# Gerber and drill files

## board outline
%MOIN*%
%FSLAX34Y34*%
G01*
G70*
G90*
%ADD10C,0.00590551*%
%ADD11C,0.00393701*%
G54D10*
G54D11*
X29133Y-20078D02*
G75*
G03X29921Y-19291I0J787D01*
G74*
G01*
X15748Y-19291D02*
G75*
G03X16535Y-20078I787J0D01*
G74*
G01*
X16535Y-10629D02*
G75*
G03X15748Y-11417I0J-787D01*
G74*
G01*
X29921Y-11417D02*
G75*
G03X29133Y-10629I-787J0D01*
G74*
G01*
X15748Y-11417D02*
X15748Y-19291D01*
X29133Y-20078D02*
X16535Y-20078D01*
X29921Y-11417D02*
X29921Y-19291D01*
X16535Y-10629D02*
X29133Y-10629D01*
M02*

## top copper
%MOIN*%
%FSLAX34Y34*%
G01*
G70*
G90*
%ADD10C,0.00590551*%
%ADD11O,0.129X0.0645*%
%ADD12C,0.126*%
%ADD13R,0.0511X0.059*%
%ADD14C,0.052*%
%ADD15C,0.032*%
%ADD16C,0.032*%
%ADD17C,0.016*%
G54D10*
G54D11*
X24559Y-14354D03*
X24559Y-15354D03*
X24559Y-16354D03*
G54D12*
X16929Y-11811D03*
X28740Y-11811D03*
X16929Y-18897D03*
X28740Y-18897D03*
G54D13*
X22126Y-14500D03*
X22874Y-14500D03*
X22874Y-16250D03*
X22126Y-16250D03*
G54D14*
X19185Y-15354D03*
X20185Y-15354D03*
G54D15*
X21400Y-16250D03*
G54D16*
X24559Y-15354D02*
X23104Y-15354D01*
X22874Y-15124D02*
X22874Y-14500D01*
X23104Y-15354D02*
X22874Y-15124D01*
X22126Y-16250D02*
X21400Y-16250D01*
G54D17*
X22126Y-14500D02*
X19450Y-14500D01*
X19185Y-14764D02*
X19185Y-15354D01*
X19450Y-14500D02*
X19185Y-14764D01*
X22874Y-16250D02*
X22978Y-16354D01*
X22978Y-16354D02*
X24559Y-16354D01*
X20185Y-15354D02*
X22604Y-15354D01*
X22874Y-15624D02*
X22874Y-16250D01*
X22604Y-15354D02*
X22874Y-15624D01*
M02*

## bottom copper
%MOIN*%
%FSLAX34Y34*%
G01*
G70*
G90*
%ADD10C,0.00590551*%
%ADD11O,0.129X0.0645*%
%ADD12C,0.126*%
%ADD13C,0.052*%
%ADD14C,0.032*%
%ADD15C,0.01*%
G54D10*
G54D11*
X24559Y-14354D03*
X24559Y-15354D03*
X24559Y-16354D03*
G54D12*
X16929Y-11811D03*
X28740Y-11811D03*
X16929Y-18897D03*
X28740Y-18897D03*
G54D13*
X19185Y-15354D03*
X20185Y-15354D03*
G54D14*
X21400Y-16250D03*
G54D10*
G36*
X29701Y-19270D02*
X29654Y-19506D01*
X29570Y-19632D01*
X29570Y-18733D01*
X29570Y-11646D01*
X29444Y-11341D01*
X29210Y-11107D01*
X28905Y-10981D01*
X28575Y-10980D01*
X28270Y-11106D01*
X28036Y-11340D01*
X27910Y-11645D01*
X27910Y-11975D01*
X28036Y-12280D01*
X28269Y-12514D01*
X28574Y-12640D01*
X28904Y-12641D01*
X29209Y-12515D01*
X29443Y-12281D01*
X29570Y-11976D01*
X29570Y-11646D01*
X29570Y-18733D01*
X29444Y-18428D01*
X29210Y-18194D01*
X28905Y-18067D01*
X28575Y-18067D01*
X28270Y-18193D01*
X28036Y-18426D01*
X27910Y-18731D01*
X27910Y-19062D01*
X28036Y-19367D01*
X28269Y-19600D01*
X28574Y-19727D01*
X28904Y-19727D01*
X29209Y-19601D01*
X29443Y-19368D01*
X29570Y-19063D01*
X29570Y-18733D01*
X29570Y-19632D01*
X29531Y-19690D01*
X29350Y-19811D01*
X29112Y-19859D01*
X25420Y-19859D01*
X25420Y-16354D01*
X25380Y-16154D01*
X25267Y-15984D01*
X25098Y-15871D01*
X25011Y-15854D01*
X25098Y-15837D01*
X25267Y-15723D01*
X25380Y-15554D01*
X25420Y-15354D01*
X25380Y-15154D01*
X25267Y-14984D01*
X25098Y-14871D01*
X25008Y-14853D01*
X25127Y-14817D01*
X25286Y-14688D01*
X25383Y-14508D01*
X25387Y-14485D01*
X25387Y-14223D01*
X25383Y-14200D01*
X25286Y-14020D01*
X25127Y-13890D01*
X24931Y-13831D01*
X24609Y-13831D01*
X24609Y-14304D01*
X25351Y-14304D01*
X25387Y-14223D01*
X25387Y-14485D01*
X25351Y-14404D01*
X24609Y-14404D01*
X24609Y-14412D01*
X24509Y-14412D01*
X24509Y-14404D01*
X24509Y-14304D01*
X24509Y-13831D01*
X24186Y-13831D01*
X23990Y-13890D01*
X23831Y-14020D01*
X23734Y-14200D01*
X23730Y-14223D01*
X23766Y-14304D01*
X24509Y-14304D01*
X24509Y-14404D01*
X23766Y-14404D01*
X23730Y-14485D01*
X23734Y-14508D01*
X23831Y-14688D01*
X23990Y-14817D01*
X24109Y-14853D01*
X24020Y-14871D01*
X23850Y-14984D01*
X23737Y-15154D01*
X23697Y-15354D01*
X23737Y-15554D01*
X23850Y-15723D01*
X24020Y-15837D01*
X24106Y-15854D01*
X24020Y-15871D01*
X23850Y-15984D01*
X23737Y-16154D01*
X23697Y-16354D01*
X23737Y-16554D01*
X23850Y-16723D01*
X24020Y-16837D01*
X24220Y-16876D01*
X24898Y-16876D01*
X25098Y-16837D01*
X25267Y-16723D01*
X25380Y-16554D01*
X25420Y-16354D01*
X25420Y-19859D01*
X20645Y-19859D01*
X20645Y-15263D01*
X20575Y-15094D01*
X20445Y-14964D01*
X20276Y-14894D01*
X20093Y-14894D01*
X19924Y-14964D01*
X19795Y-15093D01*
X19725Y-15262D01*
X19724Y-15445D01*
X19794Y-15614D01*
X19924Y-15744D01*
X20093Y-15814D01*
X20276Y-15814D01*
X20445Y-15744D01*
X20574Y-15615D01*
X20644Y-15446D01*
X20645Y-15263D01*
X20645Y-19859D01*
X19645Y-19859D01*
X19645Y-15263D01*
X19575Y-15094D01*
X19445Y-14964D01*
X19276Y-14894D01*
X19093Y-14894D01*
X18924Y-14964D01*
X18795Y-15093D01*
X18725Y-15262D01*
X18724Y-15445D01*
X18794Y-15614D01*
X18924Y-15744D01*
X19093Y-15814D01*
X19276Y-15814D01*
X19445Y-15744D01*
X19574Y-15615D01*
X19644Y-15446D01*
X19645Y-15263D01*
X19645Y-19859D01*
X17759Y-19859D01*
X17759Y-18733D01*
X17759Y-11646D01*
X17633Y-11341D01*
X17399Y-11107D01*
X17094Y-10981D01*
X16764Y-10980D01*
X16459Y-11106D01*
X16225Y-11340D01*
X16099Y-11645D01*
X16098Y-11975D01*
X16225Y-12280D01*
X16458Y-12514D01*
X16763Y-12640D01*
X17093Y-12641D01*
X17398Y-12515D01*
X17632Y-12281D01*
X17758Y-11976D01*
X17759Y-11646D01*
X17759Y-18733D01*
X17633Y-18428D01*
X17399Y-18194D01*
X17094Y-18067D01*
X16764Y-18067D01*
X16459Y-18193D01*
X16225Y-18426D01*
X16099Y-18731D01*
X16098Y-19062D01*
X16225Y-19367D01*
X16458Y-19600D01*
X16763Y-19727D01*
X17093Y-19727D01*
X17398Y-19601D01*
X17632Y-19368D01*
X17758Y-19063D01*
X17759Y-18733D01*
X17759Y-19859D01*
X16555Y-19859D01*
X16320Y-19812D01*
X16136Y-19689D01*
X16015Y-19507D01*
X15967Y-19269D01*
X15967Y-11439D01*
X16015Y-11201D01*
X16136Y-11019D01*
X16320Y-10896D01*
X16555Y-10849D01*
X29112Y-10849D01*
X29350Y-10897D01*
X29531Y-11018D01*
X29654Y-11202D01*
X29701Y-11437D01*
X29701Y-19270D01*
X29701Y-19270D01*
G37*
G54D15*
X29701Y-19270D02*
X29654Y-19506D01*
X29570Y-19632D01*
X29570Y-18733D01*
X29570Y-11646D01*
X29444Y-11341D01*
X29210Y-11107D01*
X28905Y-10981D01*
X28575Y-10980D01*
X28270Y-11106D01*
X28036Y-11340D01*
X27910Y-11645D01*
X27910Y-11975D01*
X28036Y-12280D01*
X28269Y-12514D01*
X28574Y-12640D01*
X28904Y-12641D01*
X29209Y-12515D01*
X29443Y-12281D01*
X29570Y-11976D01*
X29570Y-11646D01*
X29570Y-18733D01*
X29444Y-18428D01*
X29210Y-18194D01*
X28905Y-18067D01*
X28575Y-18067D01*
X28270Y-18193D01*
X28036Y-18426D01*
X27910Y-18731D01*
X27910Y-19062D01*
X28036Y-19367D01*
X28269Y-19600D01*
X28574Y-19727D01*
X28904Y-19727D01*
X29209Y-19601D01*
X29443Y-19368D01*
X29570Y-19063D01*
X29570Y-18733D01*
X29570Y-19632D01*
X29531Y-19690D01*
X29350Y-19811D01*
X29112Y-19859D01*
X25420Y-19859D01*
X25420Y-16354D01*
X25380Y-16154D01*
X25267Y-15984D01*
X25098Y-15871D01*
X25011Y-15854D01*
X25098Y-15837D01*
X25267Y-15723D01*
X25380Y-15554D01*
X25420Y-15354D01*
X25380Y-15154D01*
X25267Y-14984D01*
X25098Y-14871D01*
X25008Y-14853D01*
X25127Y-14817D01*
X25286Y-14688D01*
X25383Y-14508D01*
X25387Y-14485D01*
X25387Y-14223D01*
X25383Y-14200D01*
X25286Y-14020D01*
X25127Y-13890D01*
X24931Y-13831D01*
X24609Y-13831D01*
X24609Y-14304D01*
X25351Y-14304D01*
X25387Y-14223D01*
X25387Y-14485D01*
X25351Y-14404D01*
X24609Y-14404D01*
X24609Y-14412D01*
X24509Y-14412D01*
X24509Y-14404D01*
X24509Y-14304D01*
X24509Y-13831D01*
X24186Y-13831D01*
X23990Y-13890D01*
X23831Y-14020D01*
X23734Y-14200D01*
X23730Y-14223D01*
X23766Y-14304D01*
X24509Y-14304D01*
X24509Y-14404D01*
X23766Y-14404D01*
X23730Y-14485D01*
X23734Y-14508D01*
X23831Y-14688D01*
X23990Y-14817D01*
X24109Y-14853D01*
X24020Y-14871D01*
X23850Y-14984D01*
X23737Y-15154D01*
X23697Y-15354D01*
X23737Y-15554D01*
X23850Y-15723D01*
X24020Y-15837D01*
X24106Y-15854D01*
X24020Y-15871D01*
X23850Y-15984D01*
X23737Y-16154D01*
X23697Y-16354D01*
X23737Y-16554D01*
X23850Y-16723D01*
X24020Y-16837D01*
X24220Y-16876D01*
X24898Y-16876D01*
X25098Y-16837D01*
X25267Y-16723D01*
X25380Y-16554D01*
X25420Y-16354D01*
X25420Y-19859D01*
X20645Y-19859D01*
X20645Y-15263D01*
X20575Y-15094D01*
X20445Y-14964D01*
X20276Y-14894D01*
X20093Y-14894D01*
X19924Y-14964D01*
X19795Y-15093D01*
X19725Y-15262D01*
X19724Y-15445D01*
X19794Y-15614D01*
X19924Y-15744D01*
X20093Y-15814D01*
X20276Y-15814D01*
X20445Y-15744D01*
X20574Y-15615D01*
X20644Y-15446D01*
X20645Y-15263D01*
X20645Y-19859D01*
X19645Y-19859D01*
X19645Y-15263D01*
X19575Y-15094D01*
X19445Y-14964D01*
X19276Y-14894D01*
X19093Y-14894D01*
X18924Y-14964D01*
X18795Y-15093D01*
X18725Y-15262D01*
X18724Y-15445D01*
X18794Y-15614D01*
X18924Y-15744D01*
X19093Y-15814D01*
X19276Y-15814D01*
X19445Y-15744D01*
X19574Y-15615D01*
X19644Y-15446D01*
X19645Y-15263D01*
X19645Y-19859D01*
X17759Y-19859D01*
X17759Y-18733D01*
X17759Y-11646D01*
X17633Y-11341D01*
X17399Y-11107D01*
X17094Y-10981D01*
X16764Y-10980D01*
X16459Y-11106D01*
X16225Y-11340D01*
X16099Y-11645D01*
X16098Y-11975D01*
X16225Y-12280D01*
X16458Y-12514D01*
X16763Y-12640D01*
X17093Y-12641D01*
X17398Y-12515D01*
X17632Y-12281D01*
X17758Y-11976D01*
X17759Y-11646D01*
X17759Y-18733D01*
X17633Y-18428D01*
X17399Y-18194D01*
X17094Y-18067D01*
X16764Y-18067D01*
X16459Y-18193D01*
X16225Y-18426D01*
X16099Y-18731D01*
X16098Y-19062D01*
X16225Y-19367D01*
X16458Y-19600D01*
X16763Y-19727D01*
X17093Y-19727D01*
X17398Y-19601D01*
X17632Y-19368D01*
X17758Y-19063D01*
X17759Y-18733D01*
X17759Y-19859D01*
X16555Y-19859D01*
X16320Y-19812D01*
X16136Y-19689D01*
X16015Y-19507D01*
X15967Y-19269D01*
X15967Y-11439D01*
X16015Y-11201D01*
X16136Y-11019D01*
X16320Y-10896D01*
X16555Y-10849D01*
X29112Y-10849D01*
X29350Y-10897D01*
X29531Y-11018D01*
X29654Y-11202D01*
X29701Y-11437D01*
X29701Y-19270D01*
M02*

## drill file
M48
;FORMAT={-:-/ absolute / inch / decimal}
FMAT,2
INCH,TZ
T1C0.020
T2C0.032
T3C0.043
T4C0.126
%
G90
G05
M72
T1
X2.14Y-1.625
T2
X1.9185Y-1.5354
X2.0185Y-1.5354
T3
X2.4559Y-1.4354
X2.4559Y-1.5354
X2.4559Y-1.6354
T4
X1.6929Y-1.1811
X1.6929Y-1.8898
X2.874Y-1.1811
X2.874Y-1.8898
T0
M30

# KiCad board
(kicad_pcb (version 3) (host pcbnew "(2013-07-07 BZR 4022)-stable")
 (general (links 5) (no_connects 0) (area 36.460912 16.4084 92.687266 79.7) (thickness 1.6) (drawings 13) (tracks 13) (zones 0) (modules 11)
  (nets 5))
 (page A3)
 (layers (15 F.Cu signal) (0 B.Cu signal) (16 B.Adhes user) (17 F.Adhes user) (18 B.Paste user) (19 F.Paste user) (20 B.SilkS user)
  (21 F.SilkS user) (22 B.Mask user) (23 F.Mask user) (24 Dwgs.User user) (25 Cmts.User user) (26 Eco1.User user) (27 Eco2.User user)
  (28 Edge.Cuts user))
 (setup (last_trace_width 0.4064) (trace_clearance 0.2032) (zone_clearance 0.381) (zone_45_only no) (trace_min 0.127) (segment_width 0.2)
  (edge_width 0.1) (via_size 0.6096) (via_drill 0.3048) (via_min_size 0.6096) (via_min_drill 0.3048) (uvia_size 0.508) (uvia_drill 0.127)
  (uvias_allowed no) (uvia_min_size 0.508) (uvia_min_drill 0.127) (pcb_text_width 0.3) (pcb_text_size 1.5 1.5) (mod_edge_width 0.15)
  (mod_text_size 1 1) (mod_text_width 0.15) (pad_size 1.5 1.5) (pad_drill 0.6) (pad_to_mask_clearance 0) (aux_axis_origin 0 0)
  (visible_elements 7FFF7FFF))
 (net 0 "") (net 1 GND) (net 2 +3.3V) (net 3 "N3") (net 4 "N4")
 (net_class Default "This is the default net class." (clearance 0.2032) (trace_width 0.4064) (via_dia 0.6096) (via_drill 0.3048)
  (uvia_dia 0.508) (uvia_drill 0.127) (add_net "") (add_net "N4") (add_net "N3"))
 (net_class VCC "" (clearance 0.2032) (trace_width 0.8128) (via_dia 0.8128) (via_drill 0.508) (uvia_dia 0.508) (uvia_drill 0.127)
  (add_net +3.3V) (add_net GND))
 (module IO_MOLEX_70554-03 (layer F.Cu) (at 70 39 270)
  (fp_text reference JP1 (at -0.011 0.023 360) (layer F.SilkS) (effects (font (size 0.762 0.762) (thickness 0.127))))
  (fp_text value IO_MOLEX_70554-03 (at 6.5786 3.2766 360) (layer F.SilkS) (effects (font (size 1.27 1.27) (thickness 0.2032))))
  (pad 1 thru_hole oval (at -2.54 7.62 270) (size 1.6383 3.2766) (drill 1.08966) (layers *.Cu *.Adhes *.Paste *.SilkS *.Mask) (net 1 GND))
  (pad 2 thru_hole oval (at 0 7.62 270) (size 1.6383 3.2766) (drill 1.08966) (layers *.Cu *.Adhes *.Paste *.SilkS *.Mask) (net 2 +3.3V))
  (pad 3 thru_hole oval (at 2.54 7.62 270) (size 1.6383 3.2766) (drill 1.08966) (layers *.Cu *.Adhes *.Paste *.SilkS *.Mask) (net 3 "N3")))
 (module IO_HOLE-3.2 (layer F.Cu) (at 43 30)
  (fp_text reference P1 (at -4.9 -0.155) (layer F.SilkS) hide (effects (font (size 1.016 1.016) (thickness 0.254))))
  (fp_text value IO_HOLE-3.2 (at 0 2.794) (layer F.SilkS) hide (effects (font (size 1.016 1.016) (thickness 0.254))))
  (pad "" thru_hole circle (at 0 0) (size 3.2004 3.2004) (drill 3.2004) (layers *.Cu *.Paste *.SilkS *.Mask)))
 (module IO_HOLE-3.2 (layer F.Cu) (at 73 30)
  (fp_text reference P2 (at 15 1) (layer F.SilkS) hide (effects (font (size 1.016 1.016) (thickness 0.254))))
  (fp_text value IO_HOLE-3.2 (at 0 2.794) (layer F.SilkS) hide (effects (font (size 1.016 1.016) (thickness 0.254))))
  (pad "" thru_hole circle (at 0 0) (size 3.2004 3.2004) (drill 3.2004) (layers *.Cu *.Paste *.SilkS *.Mask)))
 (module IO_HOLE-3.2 (layer F.Cu) (at 43 48)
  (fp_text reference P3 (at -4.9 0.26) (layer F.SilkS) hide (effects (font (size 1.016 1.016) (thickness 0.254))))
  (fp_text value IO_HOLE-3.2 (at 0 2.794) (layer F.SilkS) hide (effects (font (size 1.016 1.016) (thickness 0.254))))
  (pad "" thru_hole circle (at 0 0) (size 3.2004 3.2004) (drill 3.2004) (layers *.Cu *.Paste *.SilkS *.Mask)))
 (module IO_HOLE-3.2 (layer F.Cu) (at 73 48)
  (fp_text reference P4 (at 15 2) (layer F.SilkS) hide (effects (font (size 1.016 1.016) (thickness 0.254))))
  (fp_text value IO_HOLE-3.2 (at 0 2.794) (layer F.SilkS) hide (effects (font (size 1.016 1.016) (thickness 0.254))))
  (pad "" thru_hole circle (at 0 0) (size 3.2004 3.2004) (drill 3.2004) (layers *.Cu *.Paste *.SilkS *.Mask)))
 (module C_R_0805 (layer F.Cu) (at 57.15 36.83)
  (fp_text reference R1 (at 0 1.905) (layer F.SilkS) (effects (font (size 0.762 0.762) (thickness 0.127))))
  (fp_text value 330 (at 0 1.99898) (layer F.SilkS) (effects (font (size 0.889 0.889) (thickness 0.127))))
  (pad 1 smd rect (at -0.94996 0) (size 1.29794 1.4986) (layers F.Cu F.Paste F.SilkS F.Mask) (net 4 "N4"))
  (pad 2 smd rect (at 0.94996 0) (size 1.29794 1.4986) (layers F.Cu F.Paste F.SilkS F.Mask) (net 2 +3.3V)))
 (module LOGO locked (layer F.Cu) (at 60.579 30.988)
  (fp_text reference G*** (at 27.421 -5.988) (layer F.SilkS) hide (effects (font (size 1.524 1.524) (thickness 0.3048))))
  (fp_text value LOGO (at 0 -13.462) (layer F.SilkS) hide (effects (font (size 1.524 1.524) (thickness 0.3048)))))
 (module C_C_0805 (layer F.Cu) (at 57.15 41.275 180)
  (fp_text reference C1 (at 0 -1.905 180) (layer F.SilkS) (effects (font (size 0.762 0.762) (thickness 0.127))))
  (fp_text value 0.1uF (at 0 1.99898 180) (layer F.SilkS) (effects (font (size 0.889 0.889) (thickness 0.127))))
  (pad 1 smd rect (at -0.94996 0 180) (size 1.29794 1.4986) (layers F.Cu F.Paste F.SilkS F.Mask) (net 3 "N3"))
  (pad 2 smd rect (at 0.94996 0 180) (size 1.29794 1.4986) (layers F.Cu F.Paste F.SilkS F.Mask) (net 1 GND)))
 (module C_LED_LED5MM (layer F.Cu) (at 50 39)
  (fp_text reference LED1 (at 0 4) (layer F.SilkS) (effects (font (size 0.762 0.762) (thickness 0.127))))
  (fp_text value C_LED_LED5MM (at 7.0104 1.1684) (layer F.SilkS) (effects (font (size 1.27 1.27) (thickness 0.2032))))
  (pad A thru_hole circle (at -1.27 0) (size 1.3208 2.6416) (drill 0.812799) (layers *.Cu *.Paste *.SilkS *.Mask) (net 4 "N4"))
  (pad K thru_hole circle (at 1.27 0) (size 1.3208 2.6416) (drill 0.812799) (layers *.Cu *.Paste *.SilkS *.Mask) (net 3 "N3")))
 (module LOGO (layer F.Cu) (at 67.056 31.242)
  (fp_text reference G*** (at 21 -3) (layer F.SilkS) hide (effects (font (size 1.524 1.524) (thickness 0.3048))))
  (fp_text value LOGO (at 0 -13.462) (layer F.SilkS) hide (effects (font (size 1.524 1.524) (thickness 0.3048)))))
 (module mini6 (layer B.Cu) (at 56 39)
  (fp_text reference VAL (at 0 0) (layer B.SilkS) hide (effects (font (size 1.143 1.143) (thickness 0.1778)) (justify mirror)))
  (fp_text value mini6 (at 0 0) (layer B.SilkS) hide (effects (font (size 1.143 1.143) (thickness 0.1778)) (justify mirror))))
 (gr_arc (start 74 49) (end 76 49) (angle 90) (layer Edge.Cuts) (width 0.1))
 (gr_arc (start 42 49) (end 42 51) (angle 90) (layer Edge.Cuts) (width 0.1))
 (gr_arc (start 42 29) (end 40 29) (angle 90) (layer Edge.Cuts) (width 0.1))
 (gr_arc (start 74 29) (end 74 27) (angle 90) (layer Edge.Cuts) (width 0.1))
 (gr_line (start 40 29) (end 40 49) (angle 90) (layer Edge.Cuts) (width 0.1))
 (gr_line (start 74 51) (end 42 51) (angle 90) (layer Edge.Cuts) (width 0.1))
 (gr_line (start 76 29) (end 76 49) (angle 90) (layer Edge.Cuts) (width 0.1))
 (gr_line (start 42 27) (end 74 27) (angle 90) (layer Edge.Cuts) (width 0.1))
 (segment (start 62.38 39) (end 58.685 39) (width 0.8128) (layer F.Cu) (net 2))
 (segment (start 58.09996 38.41496) (end 58.09996 36.83) (width 0.8128) (layer F.Cu) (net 2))
 (segment (start 58.685 39) (end 58.09996 38.41496) (width 0.8128) (layer F.Cu) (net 2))
 (segment (start 56.20004 41.275) (end 54.356 41.275) (width 0.8128) (layer F.Cu) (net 1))
 (via (at 54.356 41.275) (size 0.8128) (layers F.Cu B.Cu) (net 1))
 (segment (start 56.20004 36.83) (end 49.403 36.83) (width 0.4064) (layer F.Cu) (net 4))
 (segment (start 48.73 37.503) (end 48.73 39) (width 0.4064) (layer F.Cu) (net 4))
 (segment (start 49.403 36.83) (end 48.73 37.503) (width 0.4064) (layer F.Cu) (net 4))
 (segment (start 58.09996 41.275) (end 58.36496 41.54) (width 0.4064) (layer F.Cu) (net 3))
 (segment (start 58.36496 41.54) (end 62.38 41.54) (width 0.4064) (layer F.Cu) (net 3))
 (segment (start 51.27 39) (end 57.415 39) (width 0.4064) (layer F.Cu) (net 3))
 (segment (start 58.09996 39.68496) (end 58.09996 41.275) (width 0.4064) (layer F.Cu) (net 3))
 (segment (start 57.415 39) (end 58.09996 39.68496) (width 0.4064) (layer F.Cu) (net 3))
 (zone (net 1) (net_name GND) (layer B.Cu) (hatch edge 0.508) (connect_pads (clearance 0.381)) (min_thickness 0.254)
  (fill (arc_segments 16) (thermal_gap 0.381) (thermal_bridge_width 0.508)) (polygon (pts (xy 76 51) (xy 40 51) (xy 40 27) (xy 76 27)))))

